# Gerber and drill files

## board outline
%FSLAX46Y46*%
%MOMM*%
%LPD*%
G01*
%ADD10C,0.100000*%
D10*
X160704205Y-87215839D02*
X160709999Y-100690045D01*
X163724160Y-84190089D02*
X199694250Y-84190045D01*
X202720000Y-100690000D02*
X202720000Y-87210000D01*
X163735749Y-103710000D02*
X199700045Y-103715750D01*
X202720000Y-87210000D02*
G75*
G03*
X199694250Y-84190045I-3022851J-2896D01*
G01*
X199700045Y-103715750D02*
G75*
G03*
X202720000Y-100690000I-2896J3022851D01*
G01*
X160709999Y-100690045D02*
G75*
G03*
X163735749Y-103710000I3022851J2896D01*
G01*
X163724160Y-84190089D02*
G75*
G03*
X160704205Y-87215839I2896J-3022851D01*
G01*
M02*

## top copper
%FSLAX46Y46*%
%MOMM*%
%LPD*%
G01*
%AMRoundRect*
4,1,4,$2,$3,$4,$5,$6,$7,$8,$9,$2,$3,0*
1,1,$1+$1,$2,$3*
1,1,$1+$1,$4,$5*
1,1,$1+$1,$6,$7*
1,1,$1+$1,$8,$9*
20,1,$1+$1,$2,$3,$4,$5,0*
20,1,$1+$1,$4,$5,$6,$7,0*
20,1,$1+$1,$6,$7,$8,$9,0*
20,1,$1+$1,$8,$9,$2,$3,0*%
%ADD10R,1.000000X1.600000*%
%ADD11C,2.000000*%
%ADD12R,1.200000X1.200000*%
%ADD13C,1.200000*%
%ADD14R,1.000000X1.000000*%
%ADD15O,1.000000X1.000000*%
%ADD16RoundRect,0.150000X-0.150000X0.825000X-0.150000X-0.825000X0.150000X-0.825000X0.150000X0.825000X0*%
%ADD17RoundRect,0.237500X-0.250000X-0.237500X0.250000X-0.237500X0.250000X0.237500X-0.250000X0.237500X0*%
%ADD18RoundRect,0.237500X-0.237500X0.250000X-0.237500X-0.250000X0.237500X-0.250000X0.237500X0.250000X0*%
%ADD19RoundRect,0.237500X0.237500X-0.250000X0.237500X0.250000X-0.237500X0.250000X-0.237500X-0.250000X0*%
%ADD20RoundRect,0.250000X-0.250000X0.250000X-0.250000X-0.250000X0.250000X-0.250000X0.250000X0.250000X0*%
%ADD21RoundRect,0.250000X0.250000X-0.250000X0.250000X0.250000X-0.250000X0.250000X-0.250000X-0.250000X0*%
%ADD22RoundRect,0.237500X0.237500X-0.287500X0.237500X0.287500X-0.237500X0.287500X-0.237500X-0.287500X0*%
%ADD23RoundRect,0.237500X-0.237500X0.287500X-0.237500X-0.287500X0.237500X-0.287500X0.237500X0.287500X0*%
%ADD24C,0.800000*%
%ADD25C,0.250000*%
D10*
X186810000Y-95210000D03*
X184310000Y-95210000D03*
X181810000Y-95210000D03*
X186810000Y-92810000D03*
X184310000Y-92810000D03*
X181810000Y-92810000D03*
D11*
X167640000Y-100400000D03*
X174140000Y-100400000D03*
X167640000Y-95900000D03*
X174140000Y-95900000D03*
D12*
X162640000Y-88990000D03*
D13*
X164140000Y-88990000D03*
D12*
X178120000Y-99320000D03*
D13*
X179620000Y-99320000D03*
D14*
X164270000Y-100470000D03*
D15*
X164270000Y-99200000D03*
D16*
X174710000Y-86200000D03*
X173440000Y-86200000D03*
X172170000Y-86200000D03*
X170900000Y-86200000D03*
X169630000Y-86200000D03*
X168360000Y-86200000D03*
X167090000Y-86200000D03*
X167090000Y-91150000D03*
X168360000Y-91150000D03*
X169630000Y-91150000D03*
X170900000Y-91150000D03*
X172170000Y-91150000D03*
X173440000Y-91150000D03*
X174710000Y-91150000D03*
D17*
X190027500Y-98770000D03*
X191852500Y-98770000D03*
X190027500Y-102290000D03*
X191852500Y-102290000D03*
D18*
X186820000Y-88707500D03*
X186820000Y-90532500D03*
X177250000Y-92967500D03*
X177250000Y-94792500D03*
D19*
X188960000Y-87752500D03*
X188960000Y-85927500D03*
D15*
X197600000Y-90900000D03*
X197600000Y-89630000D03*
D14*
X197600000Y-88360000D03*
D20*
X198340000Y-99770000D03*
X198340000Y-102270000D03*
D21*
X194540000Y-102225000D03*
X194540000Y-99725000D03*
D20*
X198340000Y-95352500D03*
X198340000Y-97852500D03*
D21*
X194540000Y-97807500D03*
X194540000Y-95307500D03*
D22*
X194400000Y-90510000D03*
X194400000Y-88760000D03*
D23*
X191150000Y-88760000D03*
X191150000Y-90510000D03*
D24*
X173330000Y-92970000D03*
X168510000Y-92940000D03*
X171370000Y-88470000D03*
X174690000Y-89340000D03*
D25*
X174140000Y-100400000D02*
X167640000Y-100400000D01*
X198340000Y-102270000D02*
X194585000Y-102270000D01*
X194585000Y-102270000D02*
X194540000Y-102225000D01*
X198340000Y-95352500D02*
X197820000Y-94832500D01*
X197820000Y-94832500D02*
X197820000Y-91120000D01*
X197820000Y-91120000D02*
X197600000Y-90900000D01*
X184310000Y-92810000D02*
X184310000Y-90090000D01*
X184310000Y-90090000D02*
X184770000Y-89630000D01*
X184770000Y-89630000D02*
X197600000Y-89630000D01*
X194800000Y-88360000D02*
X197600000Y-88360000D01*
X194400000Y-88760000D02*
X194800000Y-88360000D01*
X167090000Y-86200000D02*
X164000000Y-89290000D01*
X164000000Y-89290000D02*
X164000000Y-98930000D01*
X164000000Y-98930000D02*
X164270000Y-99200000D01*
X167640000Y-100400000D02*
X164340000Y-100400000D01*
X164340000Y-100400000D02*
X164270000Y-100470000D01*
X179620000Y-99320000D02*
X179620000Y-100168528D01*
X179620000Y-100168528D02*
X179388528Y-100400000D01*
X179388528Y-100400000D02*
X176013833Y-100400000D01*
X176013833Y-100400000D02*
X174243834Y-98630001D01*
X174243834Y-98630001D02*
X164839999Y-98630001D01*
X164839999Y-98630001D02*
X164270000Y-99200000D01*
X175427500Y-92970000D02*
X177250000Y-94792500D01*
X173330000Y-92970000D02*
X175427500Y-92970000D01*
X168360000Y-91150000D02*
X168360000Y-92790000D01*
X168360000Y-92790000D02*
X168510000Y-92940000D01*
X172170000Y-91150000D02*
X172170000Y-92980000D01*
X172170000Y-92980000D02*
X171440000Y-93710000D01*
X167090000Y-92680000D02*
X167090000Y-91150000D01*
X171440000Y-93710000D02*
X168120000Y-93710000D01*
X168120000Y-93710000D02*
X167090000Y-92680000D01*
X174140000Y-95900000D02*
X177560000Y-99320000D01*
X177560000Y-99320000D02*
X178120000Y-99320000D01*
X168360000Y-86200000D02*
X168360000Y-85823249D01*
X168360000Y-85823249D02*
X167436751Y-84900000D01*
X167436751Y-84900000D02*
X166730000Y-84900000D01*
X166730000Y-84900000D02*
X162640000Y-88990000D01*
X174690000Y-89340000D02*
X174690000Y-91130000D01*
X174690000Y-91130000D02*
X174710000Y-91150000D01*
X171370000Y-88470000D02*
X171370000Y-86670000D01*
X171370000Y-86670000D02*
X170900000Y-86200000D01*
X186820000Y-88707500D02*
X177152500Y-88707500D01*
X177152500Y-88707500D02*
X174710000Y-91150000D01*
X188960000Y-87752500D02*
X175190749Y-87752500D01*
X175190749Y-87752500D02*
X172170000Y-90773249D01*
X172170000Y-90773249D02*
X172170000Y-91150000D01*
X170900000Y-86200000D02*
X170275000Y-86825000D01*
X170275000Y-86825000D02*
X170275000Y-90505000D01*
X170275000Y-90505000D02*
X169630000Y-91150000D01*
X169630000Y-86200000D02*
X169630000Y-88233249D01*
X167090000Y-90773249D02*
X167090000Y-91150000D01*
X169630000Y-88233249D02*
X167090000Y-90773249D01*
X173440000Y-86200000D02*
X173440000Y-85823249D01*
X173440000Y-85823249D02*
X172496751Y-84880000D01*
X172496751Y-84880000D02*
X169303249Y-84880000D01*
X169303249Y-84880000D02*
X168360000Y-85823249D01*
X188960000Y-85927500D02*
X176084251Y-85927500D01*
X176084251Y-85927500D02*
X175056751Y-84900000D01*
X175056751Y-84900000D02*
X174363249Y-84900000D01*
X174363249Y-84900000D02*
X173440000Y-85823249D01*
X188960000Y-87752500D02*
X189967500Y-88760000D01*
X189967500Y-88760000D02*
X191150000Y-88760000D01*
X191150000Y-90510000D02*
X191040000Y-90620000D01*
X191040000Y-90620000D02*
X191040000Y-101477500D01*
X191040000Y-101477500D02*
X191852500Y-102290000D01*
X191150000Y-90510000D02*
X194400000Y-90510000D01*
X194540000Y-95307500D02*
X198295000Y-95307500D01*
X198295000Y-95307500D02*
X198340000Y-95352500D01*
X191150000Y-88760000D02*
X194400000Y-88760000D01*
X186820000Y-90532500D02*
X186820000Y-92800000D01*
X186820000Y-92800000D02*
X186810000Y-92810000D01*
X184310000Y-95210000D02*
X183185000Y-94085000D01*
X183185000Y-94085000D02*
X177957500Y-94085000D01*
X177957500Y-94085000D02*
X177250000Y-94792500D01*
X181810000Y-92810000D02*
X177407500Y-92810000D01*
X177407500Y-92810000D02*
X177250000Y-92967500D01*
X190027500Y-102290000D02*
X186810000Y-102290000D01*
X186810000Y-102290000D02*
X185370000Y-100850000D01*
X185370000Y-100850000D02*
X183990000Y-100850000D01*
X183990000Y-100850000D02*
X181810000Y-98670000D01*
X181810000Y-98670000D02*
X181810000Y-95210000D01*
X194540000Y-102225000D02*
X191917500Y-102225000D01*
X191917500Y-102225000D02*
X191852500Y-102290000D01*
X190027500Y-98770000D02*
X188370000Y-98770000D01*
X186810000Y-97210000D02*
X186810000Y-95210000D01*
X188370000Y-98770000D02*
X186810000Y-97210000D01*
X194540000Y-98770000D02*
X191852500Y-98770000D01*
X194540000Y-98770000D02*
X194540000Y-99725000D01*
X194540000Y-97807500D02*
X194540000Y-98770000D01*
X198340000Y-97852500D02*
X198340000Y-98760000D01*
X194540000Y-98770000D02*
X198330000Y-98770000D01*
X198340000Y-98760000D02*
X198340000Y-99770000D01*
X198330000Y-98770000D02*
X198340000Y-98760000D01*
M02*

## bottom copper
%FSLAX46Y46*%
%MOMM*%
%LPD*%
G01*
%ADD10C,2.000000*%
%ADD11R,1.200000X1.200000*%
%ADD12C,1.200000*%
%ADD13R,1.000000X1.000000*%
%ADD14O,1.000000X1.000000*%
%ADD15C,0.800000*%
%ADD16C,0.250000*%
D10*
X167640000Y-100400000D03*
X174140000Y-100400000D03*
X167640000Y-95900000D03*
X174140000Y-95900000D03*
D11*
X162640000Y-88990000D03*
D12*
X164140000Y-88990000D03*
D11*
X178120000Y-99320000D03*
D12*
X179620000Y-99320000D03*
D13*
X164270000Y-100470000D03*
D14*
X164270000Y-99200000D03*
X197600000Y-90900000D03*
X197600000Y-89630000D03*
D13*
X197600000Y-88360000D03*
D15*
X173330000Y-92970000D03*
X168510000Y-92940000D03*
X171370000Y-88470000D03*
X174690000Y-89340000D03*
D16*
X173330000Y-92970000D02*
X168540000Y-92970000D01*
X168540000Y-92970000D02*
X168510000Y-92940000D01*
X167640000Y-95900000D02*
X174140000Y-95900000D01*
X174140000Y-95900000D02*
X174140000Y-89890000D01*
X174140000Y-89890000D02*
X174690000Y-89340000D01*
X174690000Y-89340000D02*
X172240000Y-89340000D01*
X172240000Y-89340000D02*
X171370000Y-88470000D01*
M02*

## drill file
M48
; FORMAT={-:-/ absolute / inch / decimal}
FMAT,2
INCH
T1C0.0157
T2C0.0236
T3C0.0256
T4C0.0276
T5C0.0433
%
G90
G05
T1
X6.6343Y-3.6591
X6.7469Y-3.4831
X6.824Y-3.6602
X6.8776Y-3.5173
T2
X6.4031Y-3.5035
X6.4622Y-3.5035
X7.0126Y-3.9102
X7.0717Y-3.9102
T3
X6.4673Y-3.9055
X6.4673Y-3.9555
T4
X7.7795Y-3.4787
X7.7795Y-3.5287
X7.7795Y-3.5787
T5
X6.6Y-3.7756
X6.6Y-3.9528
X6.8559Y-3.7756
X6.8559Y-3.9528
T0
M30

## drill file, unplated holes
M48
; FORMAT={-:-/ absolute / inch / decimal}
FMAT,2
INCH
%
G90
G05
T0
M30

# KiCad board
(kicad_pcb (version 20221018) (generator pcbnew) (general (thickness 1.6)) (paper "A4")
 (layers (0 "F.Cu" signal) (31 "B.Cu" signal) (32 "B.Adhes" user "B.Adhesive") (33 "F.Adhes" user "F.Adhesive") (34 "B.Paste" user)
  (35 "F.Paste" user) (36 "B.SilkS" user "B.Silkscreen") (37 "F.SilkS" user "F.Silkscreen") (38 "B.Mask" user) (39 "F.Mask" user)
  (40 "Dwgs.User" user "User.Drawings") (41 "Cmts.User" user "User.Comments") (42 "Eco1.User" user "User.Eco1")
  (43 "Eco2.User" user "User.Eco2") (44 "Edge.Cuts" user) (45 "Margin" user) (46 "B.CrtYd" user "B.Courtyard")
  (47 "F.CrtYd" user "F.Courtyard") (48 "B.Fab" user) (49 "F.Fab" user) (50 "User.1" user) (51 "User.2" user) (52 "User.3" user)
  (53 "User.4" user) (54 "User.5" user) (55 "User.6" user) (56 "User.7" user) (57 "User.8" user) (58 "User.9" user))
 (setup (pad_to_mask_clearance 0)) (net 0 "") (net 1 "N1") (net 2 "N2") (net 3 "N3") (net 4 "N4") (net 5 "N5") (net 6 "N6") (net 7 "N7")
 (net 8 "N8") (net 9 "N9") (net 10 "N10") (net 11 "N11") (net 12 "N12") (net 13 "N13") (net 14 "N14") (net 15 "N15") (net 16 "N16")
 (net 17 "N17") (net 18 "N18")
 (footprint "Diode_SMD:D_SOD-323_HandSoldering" (layer "F.Cu") (at 198.34 96.6025 -90)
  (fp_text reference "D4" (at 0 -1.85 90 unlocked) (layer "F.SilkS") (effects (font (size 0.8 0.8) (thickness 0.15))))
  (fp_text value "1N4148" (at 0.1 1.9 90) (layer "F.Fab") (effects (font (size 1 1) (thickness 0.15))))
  (pad "1" smd roundrect (at -1.25 0 270) (size 1 1) (layers "F.Cu" "F.Paste" "F.Mask") (roundrect_rratio 0.25) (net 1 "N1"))
  (pad "2" smd roundrect (at 1.25 0 270) (size 1 1) (layers "F.Cu" "F.Paste" "F.Mask") (roundrect_rratio 0.25) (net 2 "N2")))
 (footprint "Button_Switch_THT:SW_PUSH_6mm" (layer "F.Cu") (at 174.14 100.4 180)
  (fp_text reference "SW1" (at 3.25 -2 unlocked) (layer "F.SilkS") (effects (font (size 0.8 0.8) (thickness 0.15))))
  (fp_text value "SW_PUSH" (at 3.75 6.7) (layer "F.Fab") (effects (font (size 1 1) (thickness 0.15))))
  (pad "1" thru_hole circle (at 0 0 270) (size 2 2) (drill 1.1) (layers "*.Cu" "*.Mask") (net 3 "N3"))
  (pad "1" thru_hole circle (at 6.5 0 270) (size 2 2) (drill 1.1) (layers "*.Cu" "*.Mask") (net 3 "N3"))
  (pad "2" thru_hole circle (at 0 4.5 270) (size 2 2) (drill 1.1) (layers "*.Cu" "*.Mask") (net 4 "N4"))
  (pad "2" thru_hole circle (at 6.5 4.5 270) (size 2 2) (drill 1.1) (layers "*.Cu" "*.Mask") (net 4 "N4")))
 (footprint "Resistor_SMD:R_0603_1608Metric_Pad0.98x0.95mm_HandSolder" (layer "F.Cu") (at 190.94 98.77)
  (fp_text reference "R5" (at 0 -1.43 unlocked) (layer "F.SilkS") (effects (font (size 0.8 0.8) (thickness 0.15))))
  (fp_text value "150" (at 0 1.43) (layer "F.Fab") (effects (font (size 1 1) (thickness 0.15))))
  (pad "1" smd roundrect (at -0.9125 0) (size 0.975 0.95) (layers "F.Cu" "F.Paste" "F.Mask") (roundrect_rratio 0.25) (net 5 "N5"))
  (pad "2" smd roundrect (at 0.9125 0) (size 0.975 0.95) (layers "F.Cu" "F.Paste" "F.Mask") (roundrect_rratio 0.25) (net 2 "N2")))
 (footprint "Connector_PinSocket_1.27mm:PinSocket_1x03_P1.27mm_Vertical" (layer "F.Cu") (at 197.6 88.36)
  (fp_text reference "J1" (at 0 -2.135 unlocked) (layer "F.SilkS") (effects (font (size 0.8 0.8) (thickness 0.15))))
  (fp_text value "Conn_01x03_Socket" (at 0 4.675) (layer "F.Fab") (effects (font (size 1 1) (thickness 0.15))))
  (pad "1" thru_hole rect (at 0 0) (size 1 1) (drill 0.7) (layers "*.Cu" "*.Mask") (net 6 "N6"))
  (pad "2" thru_hole oval (at 0 1.27) (size 1 1) (drill 0.7) (layers "*.Cu" "*.Mask") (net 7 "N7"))
  (pad "3" thru_hole oval (at 0 2.54) (size 1 1) (drill 0.7) (layers "*.Cu" "*.Mask") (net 1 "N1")))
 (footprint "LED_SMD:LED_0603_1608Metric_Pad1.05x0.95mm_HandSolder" (layer "F.Cu") (at 194.4 89.635 90)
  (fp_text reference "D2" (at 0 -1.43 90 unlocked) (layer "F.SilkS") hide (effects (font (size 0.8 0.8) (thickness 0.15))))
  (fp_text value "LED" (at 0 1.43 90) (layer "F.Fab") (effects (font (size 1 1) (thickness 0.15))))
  (pad "1" smd roundrect (at -0.875 0 90) (size 1.05 0.95) (layers "F.Cu" "F.Paste" "F.Mask") (roundrect_rratio 0.25) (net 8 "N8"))
  (pad "2" smd roundrect (at 0.875 0 90) (size 1.05 0.95) (layers "F.Cu" "F.Paste" "F.Mask") (roundrect_rratio 0.25) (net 6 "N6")))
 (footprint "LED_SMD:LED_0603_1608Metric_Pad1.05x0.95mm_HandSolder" (layer "F.Cu") (at 191.15 89.635 -90)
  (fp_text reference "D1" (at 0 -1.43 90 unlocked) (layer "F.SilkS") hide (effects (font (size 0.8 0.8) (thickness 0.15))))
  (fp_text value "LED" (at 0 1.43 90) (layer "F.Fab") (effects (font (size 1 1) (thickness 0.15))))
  (pad "1" smd roundrect (at -0.875 0 270) (size 1.05 0.95) (layers "F.Cu" "F.Paste" "F.Mask") (roundrect_rratio 0.25) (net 6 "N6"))
  (pad "2" smd roundrect (at 0.875 0 270) (size 1.05 0.95) (layers "F.Cu" "F.Paste" "F.Mask") (roundrect_rratio 0.25) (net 8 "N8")))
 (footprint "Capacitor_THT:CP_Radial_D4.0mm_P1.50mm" (layer "F.Cu") (at 162.64 88.99)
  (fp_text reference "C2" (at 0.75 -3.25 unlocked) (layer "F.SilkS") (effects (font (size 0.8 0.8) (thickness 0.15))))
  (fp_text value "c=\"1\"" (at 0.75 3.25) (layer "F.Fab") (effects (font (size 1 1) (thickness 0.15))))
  (pad "1" thru_hole rect (at 0 0) (size 1.2 1.2) (drill 0.6) (layers "*.Cu" "*.Mask") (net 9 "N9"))
  (pad "2" thru_hole circle (at 1.5 0) (size 1.2 1.2) (drill 0.6) (layers "*.Cu" "*.Mask") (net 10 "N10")))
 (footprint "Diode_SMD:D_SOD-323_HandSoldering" (layer "F.Cu") (at 194.54 100.975 90)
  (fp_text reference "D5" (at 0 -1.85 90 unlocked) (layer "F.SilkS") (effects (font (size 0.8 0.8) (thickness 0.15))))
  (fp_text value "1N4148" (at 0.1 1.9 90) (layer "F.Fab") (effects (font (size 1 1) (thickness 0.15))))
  (pad "1" smd roundrect (at -1.25 0 90) (size 1 1) (layers "F.Cu" "F.Paste" "F.Mask") (roundrect_rratio 0.25) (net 8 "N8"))
  (pad "2" smd roundrect (at 1.25 0 90) (size 1 1) (layers "F.Cu" "F.Paste" "F.Mask") (roundrect_rratio 0.25) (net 2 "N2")))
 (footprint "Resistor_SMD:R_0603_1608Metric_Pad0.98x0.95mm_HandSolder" (layer "F.Cu") (at 190.94 102.29)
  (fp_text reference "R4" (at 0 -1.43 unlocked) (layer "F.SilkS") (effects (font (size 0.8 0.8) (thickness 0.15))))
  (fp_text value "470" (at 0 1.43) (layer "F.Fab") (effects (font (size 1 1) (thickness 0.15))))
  (pad "1" smd roundrect (at -0.9125 0) (size 0.975 0.95) (layers "F.Cu" "F.Paste" "F.Mask") (roundrect_rratio 0.25) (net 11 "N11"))
  (pad "2" smd roundrect (at 0.9125 0) (size 0.975 0.95) (layers "F.Cu" "F.Paste" "F.Mask") (roundrect_rratio 0.25) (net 8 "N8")))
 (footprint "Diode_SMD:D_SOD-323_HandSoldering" (layer "F.Cu") (at 194.54 96.5575 90)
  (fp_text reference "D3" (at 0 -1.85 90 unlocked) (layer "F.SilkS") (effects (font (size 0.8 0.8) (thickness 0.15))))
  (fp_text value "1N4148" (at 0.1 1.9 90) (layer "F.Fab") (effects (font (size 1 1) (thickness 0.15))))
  (pad "1" smd roundrect (at -1.25 0 90) (size 1 1) (layers "F.Cu" "F.Paste" "F.Mask") (roundrect_rratio 0.25) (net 2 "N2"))
  (pad "2" smd roundrect (at 1.25 0 90) (size 1 1) (layers "F.Cu" "F.Paste" "F.Mask") (roundrect_rratio 0.25) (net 1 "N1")))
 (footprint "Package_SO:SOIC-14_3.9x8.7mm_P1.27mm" (layer "F.Cu") (at 170.9 88.675 -90)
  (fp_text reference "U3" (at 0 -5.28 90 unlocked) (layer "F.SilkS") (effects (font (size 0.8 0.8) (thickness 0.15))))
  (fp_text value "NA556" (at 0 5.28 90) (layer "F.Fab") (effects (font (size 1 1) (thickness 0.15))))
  (pad "1" smd roundrect (at -2.475 -3.81 270) (size 1.95 0.6) (layers "F.Cu" "F.Paste" "F.Mask") (roundrect_rratio 0.25) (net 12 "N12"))
  (pad "2" smd roundrect (at -2.475 -2.54 270) (size 1.95 0.6) (layers "F.Cu" "F.Paste" "F.Mask") (roundrect_rratio 0.25) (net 9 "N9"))
  (pad "3" smd roundrect (at -2.475 -1.27 270) (size 1.95 0.6) (layers "F.Cu" "F.Paste" "F.Mask") (roundrect_rratio 0.25) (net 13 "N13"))
  (pad "4" smd roundrect (at -2.475 0 270) (size 1.95 0.6) (layers "F.Cu" "F.Paste" "F.Mask") (roundrect_rratio 0.25) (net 4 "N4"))
  (pad "5" smd roundrect (at -2.475 1.27 270) (size 1.95 0.6) (layers "F.Cu" "F.Paste" "F.Mask") (roundrect_rratio 0.25) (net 6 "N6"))
  (pad "6" smd roundrect (at -2.475 2.54 270) (size 1.95 0.6) (layers "F.Cu" "F.Paste" "F.Mask") (roundrect_rratio 0.25) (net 9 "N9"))
  (pad "7" smd roundrect (at -2.475 3.81 270) (size 1.95 0.6) (layers "F.Cu" "F.Paste" "F.Mask") (roundrect_rratio 0.25) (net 10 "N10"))
  (pad "8" smd roundrect (at 2.475 3.81 270) (size 1.95 0.6) (layers "F.Cu" "F.Paste" "F.Mask") (roundrect_rratio 0.25) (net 6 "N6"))
  (pad "9" smd roundrect (at 2.475 2.54 270) (size 1.95 0.6) (layers "F.Cu" "F.Paste" "F.Mask") (roundrect_rratio 0.25) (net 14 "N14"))
  (pad "10" smd roundrect (at 2.475 1.27 270) (size 1.95 0.6) (layers "F.Cu" "F.Paste" "F.Mask") (roundrect_rratio 0.25) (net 4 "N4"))
  (pad "11" smd roundrect (at 2.475 0 270) (size 1.95 0.6) (layers "F.Cu" "F.Paste" "F.Mask") (roundrect_rratio 0.25) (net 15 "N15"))
  (pad "12" smd roundrect (at 2.475 -1.27 270) (size 1.95 0.6) (layers "F.Cu" "F.Paste" "F.Mask") (roundrect_rratio 0.25) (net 6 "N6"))
  (pad "13" smd roundrect (at 2.475 -2.54 270) (size 1.95 0.6) (layers "F.Cu" "F.Paste" "F.Mask") (roundrect_rratio 0.25) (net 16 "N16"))
  (pad "14" smd roundrect (at 2.475 -3.81 270) (size 1.95 0.6) (layers "F.Cu" "F.Paste" "F.Mask") (roundrect_rratio 0.25) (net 4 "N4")))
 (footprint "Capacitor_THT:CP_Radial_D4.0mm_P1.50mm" (layer "F.Cu") (at 178.12 99.32)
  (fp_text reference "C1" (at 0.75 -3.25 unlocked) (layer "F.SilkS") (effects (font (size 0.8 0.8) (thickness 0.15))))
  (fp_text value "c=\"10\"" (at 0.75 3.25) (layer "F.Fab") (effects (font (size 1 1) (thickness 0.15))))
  (pad "1" thru_hole rect (at 0 0) (size 1.2 1.2) (drill 0.6) (layers "*.Cu" "*.Mask") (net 4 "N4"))
  (pad "2" thru_hole circle (at 1.5 0) (size 1.2 1.2) (drill 0.6) (layers "*.Cu" "*.Mask") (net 10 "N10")))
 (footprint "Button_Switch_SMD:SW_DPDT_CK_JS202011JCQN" (layer "F.Cu") (at 184.31 94.01 180)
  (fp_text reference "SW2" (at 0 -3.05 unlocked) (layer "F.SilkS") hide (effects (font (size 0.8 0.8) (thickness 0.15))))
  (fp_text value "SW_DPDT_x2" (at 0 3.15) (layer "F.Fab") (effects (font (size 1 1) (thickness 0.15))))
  (pad "1" smd rect (at -2.5 -1.2 180) (size 1 1.6) (layers "F.Cu" "F.Paste" "F.Mask") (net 5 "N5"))
  (pad "2" smd rect (at 0 -1.2 180) (size 1 1.6) (layers "F.Cu" "F.Paste" "F.Mask") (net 14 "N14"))
  (pad "3" smd rect (at 2.5 -1.2 180) (size 1 1.6) (layers "F.Cu" "F.Paste" "F.Mask") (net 11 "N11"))
  (pad "4" smd rect (at -2.5 1.2 180) (size 1 1.6) (layers "F.Cu" "F.Paste" "F.Mask") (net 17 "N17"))
  (pad "5" smd rect (at 0 1.2 180) (size 1 1.6) (layers "F.Cu" "F.Paste" "F.Mask") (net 7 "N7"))
  (pad "6" smd rect (at 2.5 1.2 180) (size 1 1.6) (layers "F.Cu" "F.Paste" "F.Mask") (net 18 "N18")))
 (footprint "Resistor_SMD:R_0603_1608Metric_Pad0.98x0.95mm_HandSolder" (layer "F.Cu") (at 177.25 93.88 -90)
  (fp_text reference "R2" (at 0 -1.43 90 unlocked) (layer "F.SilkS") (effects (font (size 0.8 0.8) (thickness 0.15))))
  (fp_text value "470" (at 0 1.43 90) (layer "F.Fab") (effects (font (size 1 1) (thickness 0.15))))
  (pad "1" smd roundrect (at -0.9125 0 270) (size 0.975 0.95) (layers "F.Cu" "F.Paste" "F.Mask") (roundrect_rratio 0.25) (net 18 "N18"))
  (pad "2" smd roundrect (at 0.9125 0 270) (size 0.975 0.95) (layers "F.Cu" "F.Paste" "F.Mask") (roundrect_rratio 0.25) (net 14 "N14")))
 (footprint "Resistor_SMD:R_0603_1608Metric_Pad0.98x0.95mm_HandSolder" (layer "F.Cu") (at 186.82 89.62 -90)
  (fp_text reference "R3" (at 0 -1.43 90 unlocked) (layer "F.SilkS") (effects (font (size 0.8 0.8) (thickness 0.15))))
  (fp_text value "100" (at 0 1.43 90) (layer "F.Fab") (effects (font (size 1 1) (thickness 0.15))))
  (pad "1" smd roundrect (at -0.9125 0 270) (size 0.975 0.95) (layers "F.Cu" "F.Paste" "F.Mask") (roundrect_rratio 0.25) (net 4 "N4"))
  (pad "2" smd roundrect (at 0.9125 0 270) (size 0.975 0.95) (layers "F.Cu" "F.Paste" "F.Mask") (roundrect_rratio 0.25) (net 17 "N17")))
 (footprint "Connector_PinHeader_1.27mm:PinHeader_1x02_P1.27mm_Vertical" (layer "F.Cu") (at 164.27 100.47 180)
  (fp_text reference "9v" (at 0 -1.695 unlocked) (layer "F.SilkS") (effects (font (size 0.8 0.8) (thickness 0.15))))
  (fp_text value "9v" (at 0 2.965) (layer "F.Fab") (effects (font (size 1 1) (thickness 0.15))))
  (pad "1" thru_hole rect (at 0 0 180) (size 1 1) (drill 0.65) (layers "*.Cu" "*.Mask") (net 3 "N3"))
  (pad "2" thru_hole oval (at 0 1.27 180) (size 1 1) (drill 0.65) (layers "*.Cu" "*.Mask") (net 10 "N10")))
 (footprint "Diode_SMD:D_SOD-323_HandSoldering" (layer "F.Cu") (at 198.34 101.02 -90)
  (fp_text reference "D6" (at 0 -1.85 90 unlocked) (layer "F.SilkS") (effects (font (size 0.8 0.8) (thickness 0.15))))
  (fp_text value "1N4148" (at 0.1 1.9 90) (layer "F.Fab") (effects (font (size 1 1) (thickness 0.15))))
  (pad "1" smd roundrect (at -1.25 0 270) (size 1 1) (layers "F.Cu" "F.Paste" "F.Mask") (roundrect_rratio 0.25) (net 2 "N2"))
  (pad "2" smd roundrect (at 1.25 0 270) (size 1 1) (layers "F.Cu" "F.Paste" "F.Mask") (roundrect_rratio 0.25) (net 8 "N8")))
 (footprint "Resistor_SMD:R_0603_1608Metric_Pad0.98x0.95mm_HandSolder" (layer "F.Cu") (at 188.96 86.84 90)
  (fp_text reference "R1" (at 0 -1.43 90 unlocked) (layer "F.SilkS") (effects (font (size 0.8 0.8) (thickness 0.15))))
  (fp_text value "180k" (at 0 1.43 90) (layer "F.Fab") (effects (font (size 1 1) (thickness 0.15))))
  (pad "1" smd roundrect (at -0.9125 0 90) (size 0.975 0.95) (layers "F.Cu" "F.Paste" "F.Mask") (roundrect_rratio 0.25) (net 6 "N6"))
  (pad "2" smd roundrect (at 0.9125 0 90) (size 0.975 0.95) (layers "F.Cu" "F.Paste" "F.Mask") (roundrect_rratio 0.25) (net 9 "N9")))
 (gr_arc (start 199.69425 84.190045) (mid 201.832579 85.073369) (end 202.72 87.21) (stroke (width 0.1) (type default)) (layer "Edge.Cuts"))
 (gr_arc (start 163.735749 103.71) (mid 161.59742 102.826676) (end 160.709999 100.690045) (stroke (width 0.1) (type default))
  (layer "Edge.Cuts"))
 (gr_line (start 163.735749 103.71) (end 199.700045 103.71575) (stroke (width 0.1) (type default)) (layer "Edge.Cuts"))
 (gr_line (start 160.704205 87.215839) (end 160.709999 100.690045) (stroke (width 0.1) (type default)) (layer "Edge.Cuts"))
 (gr_arc (start 202.72 100.69) (mid 201.836676 102.828329) (end 199.700045 103.71575) (stroke (width 0.1) (type default))
  (layer "Edge.Cuts"))
 (gr_line (start 202.72 100.69) (end 202.72 87.21) (stroke (width 0.1) (type default)) (layer "Edge.Cuts"))
 (gr_arc (start 160.704205 87.215839) (mid 161.587529 85.07751) (end 163.72416 84.190089) (stroke (width 0.1) (type default))
  (layer "Edge.Cuts"))
 (gr_line (start 163.72416 84.190089) (end 199.69425 84.190045) (stroke (width 0.1) (type default)) (layer "Edge.Cuts"))
 (segment (start 169.63 88.233249) (end 167.09 90.773249) (width 0.25) (layer "F.Cu") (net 6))
 (segment (start 189.9675 88.76) (end 191.15 88.76) (width 0.25) (layer "F.Cu") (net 6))
 (segment (start 191.15 88.76) (end 194.4 88.76) (width 0.25) (layer "F.Cu") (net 6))
 (segment (start 169.63 86.2) (end 169.63 88.233249) (width 0.25) (layer "F.Cu") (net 6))
 (segment (start 194.4 88.76) (end 194.8 88.36) (width 0.25) (layer "F.Cu") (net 6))
 (segment (start 175.190749 87.7525) (end 172.17 90.773249) (width 0.25) (layer "F.Cu") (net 6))
 (segment (start 167.09 92.68) (end 167.09 91.15) (width 0.25) (layer "F.Cu") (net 6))
 (segment (start 194.8 88.36) (end 197.6 88.36) (width 0.25) (layer "F.Cu") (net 6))
 (segment (start 167.09 90.773249) (end 167.09 91.15) (width 0.25) (layer "F.Cu") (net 6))
 (segment (start 172.17 91.15) (end 172.17 92.98) (width 0.25) (layer "F.Cu") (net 6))
 (segment (start 172.17 92.98) (end 171.44 93.71) (width 0.25) (layer "F.Cu") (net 6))
 (segment (start 171.44 93.71) (end 168.12 93.71) (width 0.25) (layer "F.Cu") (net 6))
 (segment (start 172.17 90.773249) (end 172.17 91.15) (width 0.25) (layer "F.Cu") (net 6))
 (segment (start 168.12 93.71) (end 167.09 92.68) (width 0.25) (layer "F.Cu") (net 6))
 (segment (start 188.96 87.7525) (end 189.9675 88.76) (width 0.25) (layer "F.Cu") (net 6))
 (segment (start 188.96 87.7525) (end 175.190749 87.7525) (width 0.25) (layer "F.Cu") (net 6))
 (segment (start 191.9175 102.225) (end 191.8525 102.29) (width 0.25) (layer "F.Cu") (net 8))
 (segment (start 191.04 101.4775) (end 191.8525 102.29) (width 0.25) (layer "F.Cu") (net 8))
 (segment (start 198.34 102.27) (end 194.585 102.27) (width 0.25) (layer "F.Cu") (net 8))
 (segment (start 191.15 90.51) (end 194.4 90.51) (width 0.25) (layer "F.Cu") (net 8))
 (segment (start 191.04 90.62) (end 191.04 101.4775) (width 0.25) (layer "F.Cu") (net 8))
 (segment (start 194.585 102.27) (end 194.54 102.225) (width 0.25) (layer "F.Cu") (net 8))
 (segment (start 194.54 102.225) (end 191.9175 102.225) (width 0.25) (layer "F.Cu") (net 8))
 (segment (start 191.15 90.51) (end 191.04 90.62) (width 0.25) (layer "F.Cu") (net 8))
 (segment (start 198.34 98.76) (end 198.34 99.77) (width 0.25) (layer "F.Cu") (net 2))
 (segment (start 194.54 98.77) (end 191.8525 98.77) (width 0.25) (layer "F.Cu") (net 2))
 (segment (start 194.54 97.8075) (end 194.54 98.77) (width 0.25) (layer "F.Cu") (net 2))
 (segment (start 198.33 98.77) (end 198.34 98.76) (width 0.25) (layer "F.Cu") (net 2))
 (segment (start 194.54 98.77) (end 194.54 99.725) (width 0.25) (layer "F.Cu") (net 2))
 (segment (start 194.54 98.77) (end 198.33 98.77) (width 0.25) (layer "F.Cu") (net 2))
 (segment (start 198.34 97.8525) (end 198.34 98.76) (width 0.25) (layer "F.Cu") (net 2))
 (segment (start 197.82 94.8325) (end 197.82 91.12) (width 0.25) (layer "F.Cu") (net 1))
 (segment (start 198.34 95.3525) (end 197.82 94.8325) (width 0.25) (layer "F.Cu") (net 1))
 (segment (start 197.82 91.12) (end 197.6 90.9) (width 0.25) (layer "F.Cu") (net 1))
 (segment (start 198.295 95.3075) (end 198.34 95.3525) (width 0.25) (layer "F.Cu") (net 1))
 (segment (start 194.54 95.3075) (end 198.295 95.3075) (width 0.25) (layer "F.Cu") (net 1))
 (segment (start 184.77 89.63) (end 197.6 89.63) (width 0.25) (layer "F.Cu") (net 7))
 (segment (start 184.31 90.09) (end 184.77 89.63) (width 0.25) (layer "F.Cu") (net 7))
 (segment (start 184.31 92.81) (end 184.31 90.09) (width 0.25) (layer "F.Cu") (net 7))
 (segment (start 175.056751 84.9) (end 174.363249 84.9) (width 0.25) (layer "F.Cu") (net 9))
 (segment (start 174.363249 84.9) (end 173.44 85.823249) (width 0.25) (layer "F.Cu") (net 9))
 (segment (start 188.96 85.9275) (end 176.084251 85.9275) (width 0.25) (layer "F.Cu") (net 9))
 (segment (start 169.303249 84.88) (end 168.36 85.823249) (width 0.25) (layer "F.Cu") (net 9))
 (segment (start 168.36 86.2) (end 168.36 85.823249) (width 0.25) (layer "F.Cu") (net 9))
 (segment (start 176.084251 85.9275) (end 175.056751 84.9) (width 0.25) (layer "F.Cu") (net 9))
 (segment (start 168.36 85.823249) (end 167.436751 84.9) (width 0.25) (layer "F.Cu") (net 9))
 (segment (start 173.44 86.2) (end 173.44 85.823249) (width 0.25) (layer "F.Cu") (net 9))
 (segment (start 173.44 85.823249) (end 172.496751 84.88) (width 0.25) (layer "F.Cu") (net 9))
 (segment (start 172.496751 84.88) (end 169.303249 84.88) (width 0.25) (layer "F.Cu") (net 9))
 (segment (start 166.73 84.9) (end 162.64 88.99) (width 0.25) (layer "F.Cu") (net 9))
 (segment (start 167.436751 84.9) (end 166.73 84.9) (width 0.25) (layer "F.Cu") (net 9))
 (segment (start 170.275 86.825) (end 170.275 90.505) (width 0.25) (layer "F.Cu") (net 4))
 (segment (start 174.14 95.9) (end 177.56 99.32) (width 0.25) (layer "F.Cu") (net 4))
 (segment (start 171.37 88.47) (end 171.37 86.67) (width 0.25) (layer "F.Cu") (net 4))
 (segment (start 174.69 91.13) (end 174.71 91.15) (width 0.25) (layer "F.Cu") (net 4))
 (segment (start 174.69 89.34) (end 174.69 91.13) (width 0.25) (layer "F.Cu") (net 4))
 (segment (start 170.9 86.2) (end 170.275 86.825) (width 0.25) (layer "F.Cu") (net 4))
 (segment (start 177.1525 88.7075) (end 174.71 91.15) (width 0.25) (layer "F.Cu") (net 4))
 (segment (start 177.56 99.32) (end 178.12 99.32) (width 0.25) (layer "F.Cu") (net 4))
 (segment (start 171.37 86.67) (end 170.9 86.2) (width 0.25) (layer "F.Cu") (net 4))
 (segment (start 170.275 90.505) (end 169.63 91.15) (width 0.25) (layer "F.Cu") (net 4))
 (segment (start 186.82 88.7075) (end 177.1525 88.7075) (width 0.25) (layer "F.Cu") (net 4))
 (via (at 174.69 89.34) (size 0.8) (drill 0.4) (layers "F.Cu" "B.Cu") (free) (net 4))
 (via (at 171.37 88.47) (size 0.8) (drill 0.4) (layers "F.Cu" "B.Cu") (free) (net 4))
 (segment (start 174.69 89.34) (end 172.24 89.34) (width 0.25) (layer "B.Cu") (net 4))
 (segment (start 167.64 95.9) (end 174.14 95.9) (width 0.25) (layer "B.Cu") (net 4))
 (segment (start 174.14 95.9) (end 174.14 89.89) (width 0.25) (layer "B.Cu") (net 4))
 (segment (start 172.24 89.34) (end 171.37 88.47) (width 0.25) (layer "B.Cu") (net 4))
 (segment (start 174.14 89.89) (end 174.69 89.34) (width 0.25) (layer "B.Cu") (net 4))
 (segment (start 179.62 99.32) (end 179.62 100.168528) (width 0.25) (layer "F.Cu") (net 10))
 (segment (start 174.243834 98.630001) (end 164.839999 98.630001) (width 0.25) (layer "F.Cu") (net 10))
 (segment (start 167.09 86.2) (end 164 89.29) (width 0.25) (layer "F.Cu") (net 10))
 (segment (start 164 98.93) (end 164.27 99.2) (width 0.25) (layer "F.Cu") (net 10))
 (segment (start 176.013833 100.4) (end 174.243834 98.630001) (width 0.25) (layer "F.Cu") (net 10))
 (segment (start 164.839999 98.630001) (end 164.27 99.2) (width 0.25) (layer "F.Cu") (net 10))
 (segment (start 179.62 100.168528) (end 179.388528 100.4) (width 0.25) (layer "F.Cu") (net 10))
 (segment (start 179.388528 100.4) (end 176.013833 100.4) (width 0.25) (layer "F.Cu") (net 10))
 (segment (start 164 89.29) (end 164 98.93) (width 0.25) (layer "F.Cu") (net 10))
 (segment (start 164.34 100.4) (end 164.27 100.47) (width 0.25) (layer "F.Cu") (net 3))
 (segment (start 167.64 100.4) (end 164.34 100.4) (width 0.25) (layer "F.Cu") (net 3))
 (segment (start 174.14 100.4) (end 167.64 100.4) (width 0.25) (layer "F.Cu") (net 3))
 (segment (start 186.82 90.5325) (end 186.82 92.8) (width 0.25) (layer "F.Cu") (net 17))
 (segment (start 186.82 92.8) (end 186.81 92.81) (width 0.25) (layer "F.Cu") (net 17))
 (segment (start 168.36 91.15) (end 168.36 92.79) (width 0.25) (layer "F.Cu") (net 14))
 (segment (start 173.33 92.97) (end 175.4275 92.97) (width 0.25) (layer "F.Cu") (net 14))
 (segment (start 184.31 95.21) (end 183.185 94.085) (width 0.25) (layer "F.Cu") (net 14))
 (segment (start 168.36 92.79) (end 168.51 92.94) (width 0.25) (layer "F.Cu") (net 14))
 (segment (start 183.185 94.085) (end 177.9575 94.085) (width 0.25) (layer "F.Cu") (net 14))
 (segment (start 177.9575 94.085) (end 177.25 94.7925) (width 0.25) (layer "F.Cu") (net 14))
 (segment (start 175.4275 92.97) (end 177.25 94.7925) (width 0.25) (layer "F.Cu") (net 14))
 (via (at 168.51 92.94) (size 0.8) (drill 0.4) (layers "F.Cu" "B.Cu") (free) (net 14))
 (via (at 173.33 92.97) (size 0.8) (drill 0.4) (layers "F.Cu" "B.Cu") (free) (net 14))
 (segment (start 168.54 92.97) (end 168.51 92.94) (width 0.25) (layer "B.Cu") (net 14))
 (segment (start 173.33 92.97) (end 168.54 92.97) (width 0.25) (layer "B.Cu") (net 14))
 (segment (start 177.4075 92.81) (end 177.25 92.9675) (width 0.25) (layer "F.Cu") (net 18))
 (segment (start 181.81 92.81) (end 177.4075 92.81) (width 0.25) (layer "F.Cu") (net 18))
 (segment (start 181.81 98.67) (end 181.81 95.21) (width 0.25) (layer "F.Cu") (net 11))
 (segment (start 183.99 100.85) (end 181.81 98.67) (width 0.25) (layer "F.Cu") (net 11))
 (segment (start 190.0275 102.29) (end 186.81 102.29) (width 0.25) (layer "F.Cu") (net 11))
 (segment (start 185.37 100.85) (end 183.99 100.85) (width 0.25) (layer "F.Cu") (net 11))
 (segment (start 186.81 102.29) (end 185.37 100.85) (width 0.25) (layer "F.Cu") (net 11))
 (segment (start 190.0275 98.77) (end 188.37 98.77) (width 0.25) (layer "F.Cu") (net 5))
 (segment (start 188.37 98.77) (end 186.81 97.21) (width 0.25) (layer "F.Cu") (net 5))
 (segment (start 186.81 97.21) (end 186.81 95.21) (width 0.25) (layer "F.Cu") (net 5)))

